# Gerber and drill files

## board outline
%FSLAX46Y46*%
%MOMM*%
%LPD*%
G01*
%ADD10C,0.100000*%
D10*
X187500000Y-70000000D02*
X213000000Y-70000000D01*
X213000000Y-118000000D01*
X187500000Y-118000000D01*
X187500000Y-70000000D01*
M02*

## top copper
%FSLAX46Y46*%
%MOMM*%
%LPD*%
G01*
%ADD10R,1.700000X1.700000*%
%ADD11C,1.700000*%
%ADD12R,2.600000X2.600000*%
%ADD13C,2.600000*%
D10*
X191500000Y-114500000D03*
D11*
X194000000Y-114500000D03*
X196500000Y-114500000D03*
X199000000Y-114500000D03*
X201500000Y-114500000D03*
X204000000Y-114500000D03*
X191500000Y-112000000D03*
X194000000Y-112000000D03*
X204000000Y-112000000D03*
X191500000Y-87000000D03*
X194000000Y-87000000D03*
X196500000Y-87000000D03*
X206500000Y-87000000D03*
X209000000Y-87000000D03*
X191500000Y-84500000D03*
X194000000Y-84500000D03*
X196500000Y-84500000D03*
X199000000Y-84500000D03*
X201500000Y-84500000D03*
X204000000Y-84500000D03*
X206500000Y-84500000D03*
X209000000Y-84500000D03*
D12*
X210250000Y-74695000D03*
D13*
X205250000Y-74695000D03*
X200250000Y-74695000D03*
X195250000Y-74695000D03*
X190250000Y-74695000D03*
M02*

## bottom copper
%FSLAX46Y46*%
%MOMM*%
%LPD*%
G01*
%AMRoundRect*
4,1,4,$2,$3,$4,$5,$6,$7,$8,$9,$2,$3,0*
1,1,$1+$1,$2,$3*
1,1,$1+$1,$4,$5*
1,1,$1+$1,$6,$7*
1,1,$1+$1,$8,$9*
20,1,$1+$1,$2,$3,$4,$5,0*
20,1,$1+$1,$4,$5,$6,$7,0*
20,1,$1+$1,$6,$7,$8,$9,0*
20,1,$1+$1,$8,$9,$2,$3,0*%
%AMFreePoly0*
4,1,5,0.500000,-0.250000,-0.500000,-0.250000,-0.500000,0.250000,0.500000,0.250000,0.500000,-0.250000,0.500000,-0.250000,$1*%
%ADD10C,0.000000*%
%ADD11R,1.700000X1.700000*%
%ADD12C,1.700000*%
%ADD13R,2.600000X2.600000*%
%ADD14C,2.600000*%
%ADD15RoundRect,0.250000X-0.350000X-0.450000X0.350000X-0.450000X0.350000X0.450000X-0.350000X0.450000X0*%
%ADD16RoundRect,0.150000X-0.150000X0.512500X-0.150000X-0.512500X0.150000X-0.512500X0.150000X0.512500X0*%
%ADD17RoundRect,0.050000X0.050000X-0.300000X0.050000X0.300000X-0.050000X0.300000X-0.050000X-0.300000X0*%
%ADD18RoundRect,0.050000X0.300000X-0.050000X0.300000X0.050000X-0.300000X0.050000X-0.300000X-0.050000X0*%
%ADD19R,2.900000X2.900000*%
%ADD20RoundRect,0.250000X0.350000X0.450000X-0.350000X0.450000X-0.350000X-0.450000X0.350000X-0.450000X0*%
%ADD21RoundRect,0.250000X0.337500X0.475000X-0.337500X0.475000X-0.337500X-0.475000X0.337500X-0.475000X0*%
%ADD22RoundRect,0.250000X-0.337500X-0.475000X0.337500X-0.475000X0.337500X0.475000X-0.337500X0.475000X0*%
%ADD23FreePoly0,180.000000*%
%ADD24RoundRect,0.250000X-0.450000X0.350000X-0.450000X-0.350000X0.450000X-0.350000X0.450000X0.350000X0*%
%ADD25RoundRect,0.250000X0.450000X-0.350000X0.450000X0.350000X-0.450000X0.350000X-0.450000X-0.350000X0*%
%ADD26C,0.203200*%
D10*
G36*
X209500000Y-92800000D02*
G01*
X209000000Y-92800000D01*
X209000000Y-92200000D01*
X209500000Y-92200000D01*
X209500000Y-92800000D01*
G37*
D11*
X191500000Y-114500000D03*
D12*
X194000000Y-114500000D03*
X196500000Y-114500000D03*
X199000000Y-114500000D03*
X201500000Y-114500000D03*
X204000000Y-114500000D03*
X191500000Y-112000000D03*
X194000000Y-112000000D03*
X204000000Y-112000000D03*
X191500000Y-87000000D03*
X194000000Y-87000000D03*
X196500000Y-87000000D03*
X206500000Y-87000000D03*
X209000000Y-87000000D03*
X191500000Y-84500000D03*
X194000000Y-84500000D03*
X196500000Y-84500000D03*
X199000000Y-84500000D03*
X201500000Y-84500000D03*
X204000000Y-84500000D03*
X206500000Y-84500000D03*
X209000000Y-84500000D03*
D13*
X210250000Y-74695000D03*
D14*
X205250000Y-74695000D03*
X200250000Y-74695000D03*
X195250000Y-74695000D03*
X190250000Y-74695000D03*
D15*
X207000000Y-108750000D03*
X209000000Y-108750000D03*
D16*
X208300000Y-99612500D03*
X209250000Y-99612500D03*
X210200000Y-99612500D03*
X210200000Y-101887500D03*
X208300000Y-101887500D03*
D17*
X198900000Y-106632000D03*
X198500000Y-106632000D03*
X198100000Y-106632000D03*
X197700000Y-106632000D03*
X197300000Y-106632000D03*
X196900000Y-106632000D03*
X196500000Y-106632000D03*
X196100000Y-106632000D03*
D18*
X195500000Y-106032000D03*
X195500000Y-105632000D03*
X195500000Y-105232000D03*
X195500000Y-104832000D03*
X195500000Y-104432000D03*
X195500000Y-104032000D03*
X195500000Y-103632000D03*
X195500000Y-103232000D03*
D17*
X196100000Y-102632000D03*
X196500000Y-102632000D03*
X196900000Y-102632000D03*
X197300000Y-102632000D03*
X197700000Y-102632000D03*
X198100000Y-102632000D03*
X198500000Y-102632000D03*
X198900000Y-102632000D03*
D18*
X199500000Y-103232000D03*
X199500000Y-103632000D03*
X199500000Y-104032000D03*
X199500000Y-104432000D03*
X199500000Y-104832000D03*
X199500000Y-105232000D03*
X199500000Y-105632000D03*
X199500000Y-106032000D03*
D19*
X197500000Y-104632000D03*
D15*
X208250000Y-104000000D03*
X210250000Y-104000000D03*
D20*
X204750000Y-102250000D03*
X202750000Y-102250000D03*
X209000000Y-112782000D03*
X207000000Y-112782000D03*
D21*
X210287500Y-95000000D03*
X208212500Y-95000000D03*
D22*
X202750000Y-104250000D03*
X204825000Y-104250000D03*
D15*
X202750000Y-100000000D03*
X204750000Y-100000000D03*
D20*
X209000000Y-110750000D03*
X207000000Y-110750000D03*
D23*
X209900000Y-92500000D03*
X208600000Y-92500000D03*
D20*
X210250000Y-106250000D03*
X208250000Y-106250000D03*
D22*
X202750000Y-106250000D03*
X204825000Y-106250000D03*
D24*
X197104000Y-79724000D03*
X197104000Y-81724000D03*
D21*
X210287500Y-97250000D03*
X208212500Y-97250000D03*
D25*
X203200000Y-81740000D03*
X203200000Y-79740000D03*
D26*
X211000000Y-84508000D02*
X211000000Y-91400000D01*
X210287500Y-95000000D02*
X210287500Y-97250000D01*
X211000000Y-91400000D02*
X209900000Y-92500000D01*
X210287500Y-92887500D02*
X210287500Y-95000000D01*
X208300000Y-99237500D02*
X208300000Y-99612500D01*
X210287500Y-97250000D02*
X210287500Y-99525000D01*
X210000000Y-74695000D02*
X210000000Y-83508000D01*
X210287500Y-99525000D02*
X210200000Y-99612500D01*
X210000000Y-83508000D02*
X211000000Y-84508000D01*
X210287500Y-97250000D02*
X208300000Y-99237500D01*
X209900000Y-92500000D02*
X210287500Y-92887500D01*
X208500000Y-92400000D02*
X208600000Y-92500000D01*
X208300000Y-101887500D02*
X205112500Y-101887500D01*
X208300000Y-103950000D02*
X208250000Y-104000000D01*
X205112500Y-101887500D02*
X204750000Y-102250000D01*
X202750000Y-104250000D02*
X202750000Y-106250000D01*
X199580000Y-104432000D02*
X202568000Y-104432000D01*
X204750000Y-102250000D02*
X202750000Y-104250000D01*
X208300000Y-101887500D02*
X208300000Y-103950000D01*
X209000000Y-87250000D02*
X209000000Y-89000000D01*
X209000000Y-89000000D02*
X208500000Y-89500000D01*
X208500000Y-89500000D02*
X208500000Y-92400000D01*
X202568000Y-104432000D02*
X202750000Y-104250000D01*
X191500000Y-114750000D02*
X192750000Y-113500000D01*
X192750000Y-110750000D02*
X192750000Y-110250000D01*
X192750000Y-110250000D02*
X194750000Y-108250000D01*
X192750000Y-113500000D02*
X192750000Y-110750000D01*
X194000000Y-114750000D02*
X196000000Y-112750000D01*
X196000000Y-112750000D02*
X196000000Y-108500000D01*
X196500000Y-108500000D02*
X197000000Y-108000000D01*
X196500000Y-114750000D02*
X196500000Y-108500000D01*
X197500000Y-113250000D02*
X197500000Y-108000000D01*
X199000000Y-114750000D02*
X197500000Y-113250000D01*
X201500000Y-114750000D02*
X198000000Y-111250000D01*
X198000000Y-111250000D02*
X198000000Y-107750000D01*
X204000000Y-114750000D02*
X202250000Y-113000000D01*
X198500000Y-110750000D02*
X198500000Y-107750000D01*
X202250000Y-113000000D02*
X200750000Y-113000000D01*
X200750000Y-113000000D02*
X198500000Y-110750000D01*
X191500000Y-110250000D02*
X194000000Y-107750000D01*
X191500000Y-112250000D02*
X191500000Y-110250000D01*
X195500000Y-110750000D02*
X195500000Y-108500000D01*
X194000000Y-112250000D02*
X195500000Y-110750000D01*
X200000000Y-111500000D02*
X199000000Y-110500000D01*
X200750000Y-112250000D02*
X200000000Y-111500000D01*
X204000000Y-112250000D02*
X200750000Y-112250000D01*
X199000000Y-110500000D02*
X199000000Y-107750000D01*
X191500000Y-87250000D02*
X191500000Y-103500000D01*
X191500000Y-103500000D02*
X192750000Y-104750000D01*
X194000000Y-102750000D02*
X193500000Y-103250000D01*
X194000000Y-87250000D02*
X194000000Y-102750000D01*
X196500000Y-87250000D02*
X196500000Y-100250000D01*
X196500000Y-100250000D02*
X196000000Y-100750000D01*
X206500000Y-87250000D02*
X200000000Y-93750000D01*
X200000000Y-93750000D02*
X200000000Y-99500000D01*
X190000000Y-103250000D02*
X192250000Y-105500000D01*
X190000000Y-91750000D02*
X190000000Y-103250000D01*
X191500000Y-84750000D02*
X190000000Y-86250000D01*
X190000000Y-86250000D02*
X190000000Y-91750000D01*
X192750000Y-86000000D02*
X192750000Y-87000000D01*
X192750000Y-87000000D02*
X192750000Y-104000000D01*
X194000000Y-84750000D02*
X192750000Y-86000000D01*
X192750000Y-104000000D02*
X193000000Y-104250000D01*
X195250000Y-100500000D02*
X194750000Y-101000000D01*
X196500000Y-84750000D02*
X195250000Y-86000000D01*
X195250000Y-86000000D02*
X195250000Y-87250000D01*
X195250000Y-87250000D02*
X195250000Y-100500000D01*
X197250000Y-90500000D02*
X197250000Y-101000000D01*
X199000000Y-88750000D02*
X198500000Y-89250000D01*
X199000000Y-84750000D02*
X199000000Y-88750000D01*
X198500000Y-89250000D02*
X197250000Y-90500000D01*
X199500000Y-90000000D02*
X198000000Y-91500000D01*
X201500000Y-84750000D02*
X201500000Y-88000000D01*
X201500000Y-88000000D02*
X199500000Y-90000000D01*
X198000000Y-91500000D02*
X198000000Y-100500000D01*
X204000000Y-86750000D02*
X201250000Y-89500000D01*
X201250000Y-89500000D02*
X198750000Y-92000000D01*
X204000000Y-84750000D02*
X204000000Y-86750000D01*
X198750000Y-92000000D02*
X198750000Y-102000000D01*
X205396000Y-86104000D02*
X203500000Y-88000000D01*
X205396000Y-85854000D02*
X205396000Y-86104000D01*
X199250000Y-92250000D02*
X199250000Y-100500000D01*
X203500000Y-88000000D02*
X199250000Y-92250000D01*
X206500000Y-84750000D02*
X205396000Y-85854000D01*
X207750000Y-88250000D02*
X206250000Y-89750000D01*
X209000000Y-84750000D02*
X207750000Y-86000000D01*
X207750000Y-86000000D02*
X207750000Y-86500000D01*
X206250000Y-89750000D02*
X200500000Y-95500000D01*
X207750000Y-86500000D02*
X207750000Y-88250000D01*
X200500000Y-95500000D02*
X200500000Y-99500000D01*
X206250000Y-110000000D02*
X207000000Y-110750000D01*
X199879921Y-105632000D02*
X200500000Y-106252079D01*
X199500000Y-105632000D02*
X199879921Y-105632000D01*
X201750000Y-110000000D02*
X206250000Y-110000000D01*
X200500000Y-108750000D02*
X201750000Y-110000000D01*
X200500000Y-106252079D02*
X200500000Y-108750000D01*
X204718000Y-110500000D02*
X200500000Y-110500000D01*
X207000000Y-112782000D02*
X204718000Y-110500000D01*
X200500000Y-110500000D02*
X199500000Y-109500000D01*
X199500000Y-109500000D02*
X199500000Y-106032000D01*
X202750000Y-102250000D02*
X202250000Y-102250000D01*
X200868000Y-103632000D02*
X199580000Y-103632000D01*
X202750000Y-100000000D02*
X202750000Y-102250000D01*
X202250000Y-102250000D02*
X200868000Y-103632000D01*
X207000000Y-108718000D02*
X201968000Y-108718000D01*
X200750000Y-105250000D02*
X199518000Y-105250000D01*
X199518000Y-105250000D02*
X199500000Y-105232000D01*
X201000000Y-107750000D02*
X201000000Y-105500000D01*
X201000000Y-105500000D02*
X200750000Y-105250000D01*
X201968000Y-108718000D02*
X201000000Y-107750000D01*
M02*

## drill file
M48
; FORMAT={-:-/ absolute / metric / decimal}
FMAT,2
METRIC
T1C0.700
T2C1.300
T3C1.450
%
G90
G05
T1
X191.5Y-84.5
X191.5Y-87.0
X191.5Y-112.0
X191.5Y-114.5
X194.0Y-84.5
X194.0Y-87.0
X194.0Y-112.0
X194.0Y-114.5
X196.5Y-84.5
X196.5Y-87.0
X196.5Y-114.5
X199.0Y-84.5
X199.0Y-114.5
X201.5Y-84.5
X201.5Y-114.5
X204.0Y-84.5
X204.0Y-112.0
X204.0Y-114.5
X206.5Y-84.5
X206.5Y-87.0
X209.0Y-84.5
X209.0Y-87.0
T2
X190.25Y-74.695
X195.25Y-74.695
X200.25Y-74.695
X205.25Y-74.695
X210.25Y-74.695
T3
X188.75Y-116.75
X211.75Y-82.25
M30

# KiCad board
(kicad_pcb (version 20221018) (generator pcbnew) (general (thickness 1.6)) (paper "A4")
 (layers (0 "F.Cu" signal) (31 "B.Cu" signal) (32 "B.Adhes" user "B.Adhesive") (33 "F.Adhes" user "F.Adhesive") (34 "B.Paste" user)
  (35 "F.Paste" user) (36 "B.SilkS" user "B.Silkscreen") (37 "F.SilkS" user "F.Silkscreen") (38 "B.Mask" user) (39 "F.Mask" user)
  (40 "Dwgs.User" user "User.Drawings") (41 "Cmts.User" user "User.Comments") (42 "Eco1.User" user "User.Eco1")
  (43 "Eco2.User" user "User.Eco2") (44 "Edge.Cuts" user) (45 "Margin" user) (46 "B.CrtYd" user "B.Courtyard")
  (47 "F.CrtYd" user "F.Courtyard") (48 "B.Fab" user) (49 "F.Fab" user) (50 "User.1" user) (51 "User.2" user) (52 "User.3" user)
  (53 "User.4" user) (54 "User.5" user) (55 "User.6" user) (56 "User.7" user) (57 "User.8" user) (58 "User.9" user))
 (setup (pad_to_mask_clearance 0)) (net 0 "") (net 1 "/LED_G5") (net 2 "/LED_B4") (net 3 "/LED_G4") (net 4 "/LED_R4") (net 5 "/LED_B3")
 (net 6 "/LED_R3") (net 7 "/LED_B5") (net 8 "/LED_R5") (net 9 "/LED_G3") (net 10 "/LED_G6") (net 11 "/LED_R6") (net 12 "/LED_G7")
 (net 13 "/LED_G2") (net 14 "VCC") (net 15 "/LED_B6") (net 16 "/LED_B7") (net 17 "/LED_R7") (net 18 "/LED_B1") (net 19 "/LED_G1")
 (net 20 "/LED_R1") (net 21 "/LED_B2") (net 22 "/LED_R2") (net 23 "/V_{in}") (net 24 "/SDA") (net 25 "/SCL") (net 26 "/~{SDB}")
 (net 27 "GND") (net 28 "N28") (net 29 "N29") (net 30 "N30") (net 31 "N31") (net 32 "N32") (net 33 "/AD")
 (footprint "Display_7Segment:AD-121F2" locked (layer "F.Cu") (at 191.5 114.5 90)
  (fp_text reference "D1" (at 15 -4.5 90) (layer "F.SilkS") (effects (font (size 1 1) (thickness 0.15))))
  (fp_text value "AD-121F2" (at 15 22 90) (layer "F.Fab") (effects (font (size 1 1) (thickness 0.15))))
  (pad "" np_thru_hole circle locked (at -2.25 -2.75 90) (size 1.45 1.45) (drill 1.45) (layers "*.Cu" "*.Mask"))
  (pad "" np_thru_hole circle locked (at 32.25 20.25 90) (size 1.45 1.45) (drill 1.45) (layers "*.Cu" "*.Mask"))
  (pad "1" thru_hole rect locked (at 0 0 90) (size 1.7 1.7) (drill 0.7) (layers "*.Cu" "*.Mask") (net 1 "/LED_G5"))
  (pad "2" thru_hole circle locked (at 0 2.5 90) (size 1.7 1.7) (drill 0.7) (layers "*.Cu" "*.Mask") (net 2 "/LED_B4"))
  (pad "3" thru_hole circle locked (at 0 5 90) (size 1.7 1.7) (drill 0.7) (layers "*.Cu" "*.Mask") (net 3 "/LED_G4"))
  (pad "4" thru_hole circle locked (at 0 7.5 90) (size 1.7 1.7) (drill 0.7) (layers "*.Cu" "*.Mask") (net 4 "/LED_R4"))
  (pad "5" thru_hole circle locked (at 0 10 90) (size 1.7 1.7) (drill 0.7) (layers "*.Cu" "*.Mask") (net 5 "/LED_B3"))
  (pad "6" thru_hole circle locked (at 0 12.5 90) (size 1.7 1.7) (drill 0.7) (layers "*.Cu" "*.Mask") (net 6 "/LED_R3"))
  (pad "9" thru_hole circle locked (at 2.5 0 90) (size 1.7 1.7) (drill 0.7) (layers "*.Cu" "*.Mask") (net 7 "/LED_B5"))
  (pad "10" thru_hole circle locked (at 2.5 2.5 90) (size 1.7 1.7) (drill 0.7) (layers "*.Cu" "*.Mask") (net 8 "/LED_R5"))
  (pad "11" thru_hole circle locked (at 2.5 12.5 90) (size 1.7 1.7) (drill 0.7) (layers "*.Cu" "*.Mask") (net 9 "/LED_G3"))
  (pad "13" thru_hole circle locked (at 27.5 0 90) (size 1.7 1.7) (drill 0.7) (layers "*.Cu" "*.Mask") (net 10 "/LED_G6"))
  (pad "14" thru_hole circle locked (at 27.5 2.5 90) (size 1.7 1.7) (drill 0.7) (layers "*.Cu" "*.Mask") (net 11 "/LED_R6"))
  (pad "15" thru_hole circle locked (at 27.5 5 90) (size 1.7 1.7) (drill 0.7) (layers "*.Cu" "*.Mask") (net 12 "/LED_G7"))
  (pad "16" thru_hole circle locked (at 27.5 15 90) (size 1.7 1.7) (drill 0.7) (layers "*.Cu" "*.Mask") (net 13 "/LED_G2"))
  (pad "17" thru_hole circle locked (at 27.5 17.5 90) (size 1.7 1.7) (drill 0.7) (layers "*.Cu" "*.Mask") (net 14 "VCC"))
  (pad "18" thru_hole circle locked (at 30 0 90) (size 1.7 1.7) (drill 0.7) (layers "*.Cu" "*.Mask") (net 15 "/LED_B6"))
  (pad "19" thru_hole circle locked (at 30 2.5 90) (size 1.7 1.7) (drill 0.7) (layers "*.Cu" "*.Mask") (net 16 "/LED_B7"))
  (pad "20" thru_hole circle locked (at 30 5 90) (size 1.7 1.7) (drill 0.7) (layers "*.Cu" "*.Mask") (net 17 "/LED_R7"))
  (pad "21" thru_hole circle locked (at 30 7.5 90) (size 1.7 1.7) (drill 0.7) (layers "*.Cu" "*.Mask") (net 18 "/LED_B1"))
  (pad "22" thru_hole circle locked (at 30 10 90) (size 1.7 1.7) (drill 0.7) (layers "*.Cu" "*.Mask") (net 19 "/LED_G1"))
  (pad "23" thru_hole circle locked (at 30 12.5 90) (size 1.7 1.7) (drill 0.7) (layers "*.Cu" "*.Mask") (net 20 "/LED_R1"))
  (pad "24" thru_hole circle locked (at 30 15 90) (size 1.7 1.7) (drill 0.7) (layers "*.Cu" "*.Mask") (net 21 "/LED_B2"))
  (pad "25" thru_hole circle locked (at 30 17.5 90) (size 1.7 1.7) (drill 0.7) (layers "*.Cu" "*.Mask") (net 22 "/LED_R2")))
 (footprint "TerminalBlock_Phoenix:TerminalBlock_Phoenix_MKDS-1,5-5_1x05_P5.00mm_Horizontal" (layer "F.Cu") (at 210.25 74.695 180)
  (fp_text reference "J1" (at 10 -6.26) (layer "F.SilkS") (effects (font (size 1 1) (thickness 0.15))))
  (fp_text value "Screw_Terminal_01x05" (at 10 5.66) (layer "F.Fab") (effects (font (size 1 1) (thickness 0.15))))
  (pad "1" thru_hole rect (at 0 0 180) (size 2.6 2.6) (drill 1.3) (layers "*.Cu" "*.Mask") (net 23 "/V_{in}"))
  (pad "2" thru_hole circle (at 5 0 180) (size 2.6 2.6) (drill 1.3) (layers "*.Cu" "*.Mask") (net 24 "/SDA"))
  (pad "3" thru_hole circle (at 10 0 180) (size 2.6 2.6) (drill 1.3) (layers "*.Cu" "*.Mask") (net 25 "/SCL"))
  (pad "4" thru_hole circle (at 15 0 180) (size 2.6 2.6) (drill 1.3) (layers "*.Cu" "*.Mask") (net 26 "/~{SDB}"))
  (pad "5" thru_hole circle (at 20 0 180) (size 2.6 2.6) (drill 1.3) (layers "*.Cu" "*.Mask") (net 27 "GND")))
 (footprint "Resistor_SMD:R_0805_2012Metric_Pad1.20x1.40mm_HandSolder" (layer "B.Cu") (at 208 108.75)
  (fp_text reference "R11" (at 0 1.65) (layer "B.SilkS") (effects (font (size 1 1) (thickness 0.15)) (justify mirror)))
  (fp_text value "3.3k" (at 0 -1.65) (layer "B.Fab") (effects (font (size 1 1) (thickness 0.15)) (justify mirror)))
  (pad "1" smd roundrect (at -1 0) (size 1.2 1.4) (layers "B.Cu" "B.Paste" "B.Mask") (roundrect_rratio 0.208333) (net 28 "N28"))
  (pad "2" smd roundrect (at 1 0) (size 1.2 1.4) (layers "B.Cu" "B.Paste" "B.Mask") (roundrect_rratio 0.208333) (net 27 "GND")))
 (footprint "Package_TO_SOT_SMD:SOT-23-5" (layer "B.Cu") (at 209.25 100.75 -90)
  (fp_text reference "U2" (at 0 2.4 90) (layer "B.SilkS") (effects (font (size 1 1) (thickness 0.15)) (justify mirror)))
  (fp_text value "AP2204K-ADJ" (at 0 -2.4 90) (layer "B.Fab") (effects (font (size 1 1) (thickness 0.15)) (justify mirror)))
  (pad "1" smd roundrect (at -1.1375 0.95 270) (size 1.325 0.6) (layers "B.Cu" "B.Paste" "B.Mask") (roundrect_rratio 0.25)
   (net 23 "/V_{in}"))
  (pad "2" smd roundrect (at -1.1375 0 270) (size 1.325 0.6) (layers "B.Cu" "B.Paste" "B.Mask") (roundrect_rratio 0.25) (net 27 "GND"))
  (pad "3" smd roundrect (at -1.1375 -0.95 270) (size 1.325 0.6) (layers "B.Cu" "B.Paste" "B.Mask") (roundrect_rratio 0.25)
   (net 23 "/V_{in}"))
  (pad "4" smd roundrect (at 1.1375 -0.95 270) (size 1.325 0.6) (layers "B.Cu" "B.Paste" "B.Mask") (roundrect_rratio 0.25) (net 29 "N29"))
  (pad "5" smd roundrect (at 1.1375 0.95 270) (size 1.325 0.6) (layers "B.Cu" "B.Paste" "B.Mask") (roundrect_rratio 0.25) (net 14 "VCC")))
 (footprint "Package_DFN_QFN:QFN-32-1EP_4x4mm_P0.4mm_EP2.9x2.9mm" (layer "B.Cu") (at 197.5 104.632 90)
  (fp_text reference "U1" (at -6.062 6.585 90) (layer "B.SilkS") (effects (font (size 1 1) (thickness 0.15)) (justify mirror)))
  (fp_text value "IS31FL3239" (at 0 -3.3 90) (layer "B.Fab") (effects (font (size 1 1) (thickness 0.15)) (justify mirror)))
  (pad "" smd roundrect (at -0.725 -0.725 90) (size 1.17 1.17) (layers "B.Paste") (roundrect_rratio 0.213675))
  (pad "" smd roundrect (at -0.725 0.725 90) (size 1.17 1.17) (layers "B.Paste") (roundrect_rratio 0.213675))
  (pad "" smd roundrect (at 0.725 -0.725 90) (size 1.17 1.17) (layers "B.Paste") (roundrect_rratio 0.213675))
  (pad "" smd roundrect (at 0.725 0.725 90) (size 1.17 1.17) (layers "B.Paste") (roundrect_rratio 0.213675))
  (pad "1" smd roundrect (at -2 1.4 90) (size 0.7 0.2) (layers "B.Cu" "B.Paste" "B.Mask") (roundrect_rratio 0.25) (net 20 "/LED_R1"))
  (pad "2" smd roundrect (at -2 1 90) (size 0.7 0.2) (layers "B.Cu" "B.Paste" "B.Mask") (roundrect_rratio 0.25) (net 19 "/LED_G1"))
  (pad "3" smd roundrect (at -2 0.6 90) (size 0.7 0.2) (layers "B.Cu" "B.Paste" "B.Mask") (roundrect_rratio 0.25) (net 18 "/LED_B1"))
  (pad "4" smd roundrect (at -2 0.2 90) (size 0.7 0.2) (layers "B.Cu" "B.Paste" "B.Mask") (roundrect_rratio 0.25) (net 22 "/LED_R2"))
  (pad "5" smd roundrect (at -2 -0.2 90) (size 0.7 0.2) (layers "B.Cu" "B.Paste" "B.Mask") (roundrect_rratio 0.25) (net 13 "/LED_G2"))
  (pad "6" smd roundrect (at -2 -0.6 90) (size 0.7 0.2) (layers "B.Cu" "B.Paste" "B.Mask") (roundrect_rratio 0.25) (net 21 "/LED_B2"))
  (pad "7" smd roundrect (at -2 -1 90) (size 0.7 0.2) (layers "B.Cu" "B.Paste" "B.Mask") (roundrect_rratio 0.25) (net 6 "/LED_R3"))
  (pad "8" smd roundrect (at -2 -1.4 90) (size 0.7 0.2) (layers "B.Cu" "B.Paste" "B.Mask") (roundrect_rratio 0.25) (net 9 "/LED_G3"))
  (pad "9" smd roundrect (at -1.4 -2 90) (size 0.2 0.7) (layers "B.Cu" "B.Paste" "B.Mask") (roundrect_rratio 0.25) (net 5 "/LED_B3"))
  (pad "10" smd roundrect (at -1 -2 90) (size 0.2 0.7) (layers "B.Cu" "B.Paste" "B.Mask") (roundrect_rratio 0.25) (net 4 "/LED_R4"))
  (pad "11" smd roundrect (at -0.6 -2 90) (size 0.2 0.7) (layers "B.Cu" "B.Paste" "B.Mask") (roundrect_rratio 0.25) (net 3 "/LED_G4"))
  (pad "12" smd roundrect (at -0.2 -2 90) (size 0.2 0.7) (layers "B.Cu" "B.Paste" "B.Mask") (roundrect_rratio 0.25) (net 2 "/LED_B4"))
  (pad "13" smd roundrect (at 0.2 -2 90) (size 0.2 0.7) (layers "B.Cu" "B.Paste" "B.Mask") (roundrect_rratio 0.25) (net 27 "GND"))
  (pad "14" smd roundrect (at 0.6 -2 90) (size 0.2 0.7) (layers "B.Cu" "B.Paste" "B.Mask") (roundrect_rratio 0.25) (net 8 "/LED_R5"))
  (pad "15" smd roundrect (at 1 -2 90) (size 0.2 0.7) (layers "B.Cu" "B.Paste" "B.Mask") (roundrect_rratio 0.25) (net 1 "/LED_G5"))
  (pad "16" smd roundrect (at 1.4 -2 90) (size 0.2 0.7) (layers "B.Cu" "B.Paste" "B.Mask") (roundrect_rratio 0.25) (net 7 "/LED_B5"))
  (pad "17" smd roundrect (at 2 -1.4 90) (size 0.7 0.2) (layers "B.Cu" "B.Paste" "B.Mask") (roundrect_rratio 0.25) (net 11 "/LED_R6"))
  (pad "18" smd roundrect (at 2 -1 90) (size 0.7 0.2) (layers "B.Cu" "B.Paste" "B.Mask") (roundrect_rratio 0.25) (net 10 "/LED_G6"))
  (pad "19" smd roundrect (at 2 -0.6 90) (size 0.7 0.2) (layers "B.Cu" "B.Paste" "B.Mask") (roundrect_rratio 0.25) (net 15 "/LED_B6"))
  (pad "20" smd roundrect (at 2 -0.2 90) (size 0.7 0.2) (layers "B.Cu" "B.Paste" "B.Mask") (roundrect_rratio 0.25) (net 17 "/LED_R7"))
  (pad "21" smd roundrect (at 2 0.2 90) (size 0.7 0.2) (layers "B.Cu" "B.Paste" "B.Mask") (roundrect_rratio 0.25) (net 12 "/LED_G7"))
  (pad "22" smd roundrect (at 2 0.6 90) (size 0.7 0.2) (layers "B.Cu" "B.Paste" "B.Mask") (roundrect_rratio 0.25) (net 16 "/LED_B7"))
  (pad "23" smd roundrect (at 2 1 90) (size 0.7 0.2) (layers "B.Cu" "B.Paste" "B.Mask") (roundrect_rratio 0.25) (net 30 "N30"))
  (pad "24" smd roundrect (at 2 1.4 90) (size 0.7 0.2) (layers "B.Cu" "B.Paste" "B.Mask") (roundrect_rratio 0.25) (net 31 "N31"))
  (pad "25" smd roundrect (at 1.4 2 90) (size 0.2 0.7) (layers "B.Cu" "B.Paste" "B.Mask") (roundrect_rratio 0.25) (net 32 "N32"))
  (pad "26" smd roundrect (at 1 2 90) (size 0.2 0.7) (layers "B.Cu" "B.Paste" "B.Mask") (roundrect_rratio 0.25) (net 26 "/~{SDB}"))
  (pad "27" smd roundrect (at 0.6 2 90) (size 0.2 0.7) (layers "B.Cu" "B.Paste" "B.Mask") (roundrect_rratio 0.25) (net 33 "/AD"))
  (pad "28" smd roundrect (at 0.2 2 90) (size 0.2 0.7) (layers "B.Cu" "B.Paste" "B.Mask") (roundrect_rratio 0.25) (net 14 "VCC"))
  (pad "29" smd roundrect (at -0.2 2 90) (size 0.2 0.7) (layers "B.Cu" "B.Paste" "B.Mask") (roundrect_rratio 0.25) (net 27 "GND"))
  (pad "30" smd roundrect (at -0.6 2 90) (size 0.2 0.7) (layers "B.Cu" "B.Paste" "B.Mask") (roundrect_rratio 0.25) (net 28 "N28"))
  (pad "31" smd roundrect (at -1 2 90) (size 0.2 0.7) (layers "B.Cu" "B.Paste" "B.Mask") (roundrect_rratio 0.25) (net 24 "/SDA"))
  (pad "32" smd roundrect (at -1.4 2 90) (size 0.2 0.7) (layers "B.Cu" "B.Paste" "B.Mask") (roundrect_rratio 0.25) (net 25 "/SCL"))
  (pad "33" smd rect (at 0 0 90) (size 2.9 2.9) (layers "B.Cu" "B.Mask") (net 27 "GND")))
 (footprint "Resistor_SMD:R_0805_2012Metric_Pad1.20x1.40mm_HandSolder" (layer "B.Cu") (at 209.25 104)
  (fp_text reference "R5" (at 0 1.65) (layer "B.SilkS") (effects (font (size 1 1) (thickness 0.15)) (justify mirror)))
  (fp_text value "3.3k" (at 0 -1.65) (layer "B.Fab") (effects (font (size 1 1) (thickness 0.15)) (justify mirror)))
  (pad "1" smd roundrect (at -1 0) (size 1.2 1.4) (layers "B.Cu" "B.Paste" "B.Mask") (roundrect_rratio 0.208333) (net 14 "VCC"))
  (pad "2" smd roundrect (at 1 0) (size 1.2 1.4) (layers "B.Cu" "B.Paste" "B.Mask") (roundrect_rratio 0.208333) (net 29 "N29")))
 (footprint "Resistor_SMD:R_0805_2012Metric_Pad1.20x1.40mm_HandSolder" (layer "B.Cu") (at 203.75 102.25 180)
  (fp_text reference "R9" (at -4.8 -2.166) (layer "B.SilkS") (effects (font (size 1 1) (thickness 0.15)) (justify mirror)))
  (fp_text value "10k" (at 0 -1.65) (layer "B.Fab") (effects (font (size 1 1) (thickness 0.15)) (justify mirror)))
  (pad "1" smd roundrect (at -1 0 180) (size 1.2 1.4) (layers "B.Cu" "B.Paste" "B.Mask") (roundrect_rratio 0.208333) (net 14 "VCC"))
  (pad "2" smd roundrect (at 1 0 180) (size 1.2 1.4) (layers "B.Cu" "B.Paste" "B.Mask") (roundrect_rratio 0.208333) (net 26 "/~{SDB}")))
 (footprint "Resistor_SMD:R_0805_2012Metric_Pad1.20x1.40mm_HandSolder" (layer "B.Cu") (at 208 112.782 180)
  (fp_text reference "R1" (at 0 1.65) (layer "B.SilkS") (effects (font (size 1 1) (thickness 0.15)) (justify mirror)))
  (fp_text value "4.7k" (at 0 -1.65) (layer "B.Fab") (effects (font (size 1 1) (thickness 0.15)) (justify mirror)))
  (pad "1" smd roundrect (at -1 0 180) (size 1.2 1.4) (layers "B.Cu" "B.Paste" "B.Mask") (roundrect_rratio 0.208333) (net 14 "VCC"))
  (pad "2" smd roundrect (at 1 0 180) (size 1.2 1.4) (layers "B.Cu" "B.Paste" "B.Mask") (roundrect_rratio 0.208333) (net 25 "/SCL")))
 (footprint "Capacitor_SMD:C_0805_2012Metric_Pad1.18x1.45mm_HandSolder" (layer "B.Cu") (at 209.25 95 180)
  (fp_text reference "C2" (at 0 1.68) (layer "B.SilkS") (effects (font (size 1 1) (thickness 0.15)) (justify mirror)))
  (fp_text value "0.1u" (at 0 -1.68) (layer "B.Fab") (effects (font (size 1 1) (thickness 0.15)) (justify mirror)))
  (pad "1" smd roundrect (at -1.0375 0 180) (size 1.175 1.45) (layers "B.Cu" "B.Paste" "B.Mask") (roundrect_rratio 0.212766)
   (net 23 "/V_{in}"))
  (pad "2" smd roundrect (at 1.0375 0 180) (size 1.175 1.45) (layers "B.Cu" "B.Paste" "B.Mask") (roundrect_rratio 0.212766) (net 27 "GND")))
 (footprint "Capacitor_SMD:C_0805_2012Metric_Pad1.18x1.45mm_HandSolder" (layer "B.Cu") (at 203.7875 104.25)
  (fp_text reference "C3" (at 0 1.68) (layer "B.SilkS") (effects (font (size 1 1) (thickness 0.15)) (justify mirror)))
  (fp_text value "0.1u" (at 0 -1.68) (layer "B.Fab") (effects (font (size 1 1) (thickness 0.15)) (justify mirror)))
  (pad "1" smd roundrect (at -1.0375 0) (size 1.175 1.45) (layers "B.Cu" "B.Paste" "B.Mask") (roundrect_rratio 0.212766) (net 14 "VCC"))
  (pad "2" smd roundrect (at 1.0375 0) (size 1.175 1.45) (layers "B.Cu" "B.Paste" "B.Mask") (roundrect_rratio 0.212766) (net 27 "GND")))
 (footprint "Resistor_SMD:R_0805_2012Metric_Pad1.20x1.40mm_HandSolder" (layer "B.Cu") (at 203.75 100)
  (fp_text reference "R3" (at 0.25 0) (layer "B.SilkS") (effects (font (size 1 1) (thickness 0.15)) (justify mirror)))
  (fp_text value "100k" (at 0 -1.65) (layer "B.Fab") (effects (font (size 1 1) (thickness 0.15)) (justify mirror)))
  (pad "1" smd roundrect (at -1 0) (size 1.2 1.4) (layers "B.Cu" "B.Paste" "B.Mask") (roundrect_rratio 0.208333) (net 26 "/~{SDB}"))
  (pad "2" smd roundrect (at 1 0) (size 1.2 1.4) (layers "B.Cu" "B.Paste" "B.Mask") (roundrect_rratio 0.208333) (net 27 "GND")))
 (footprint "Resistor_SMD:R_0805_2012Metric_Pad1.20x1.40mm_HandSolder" (layer "B.Cu") (at 208 110.75 180)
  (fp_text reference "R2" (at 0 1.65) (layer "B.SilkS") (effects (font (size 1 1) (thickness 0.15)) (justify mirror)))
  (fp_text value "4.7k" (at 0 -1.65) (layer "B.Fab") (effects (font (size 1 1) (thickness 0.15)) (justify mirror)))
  (pad "1" smd roundrect (at -1 0 180) (size 1.2 1.4) (layers "B.Cu" "B.Paste" "B.Mask") (roundrect_rratio 0.208333) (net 14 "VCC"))
  (pad "2" smd roundrect (at 1 0 180) (size 1.2 1.4) (layers "B.Cu" "B.Paste" "B.Mask") (roundrect_rratio 0.208333) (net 24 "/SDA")))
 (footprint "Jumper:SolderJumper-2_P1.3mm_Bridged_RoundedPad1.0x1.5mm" (layer "B.Cu") (at 209.25 92.5 180) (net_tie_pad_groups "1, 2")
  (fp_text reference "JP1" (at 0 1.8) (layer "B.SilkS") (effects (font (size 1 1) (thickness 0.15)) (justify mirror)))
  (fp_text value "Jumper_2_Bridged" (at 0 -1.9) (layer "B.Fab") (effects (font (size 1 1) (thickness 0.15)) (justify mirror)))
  (fp_poly (pts (xy 0.25 0.3) (xy -0.25 0.3) (xy -0.25 -0.3) (xy 0.25 -0.3)) (stroke (width 0) (type solid)) (fill solid) (layer "B.Cu"))
  (pad "1" smd custom (at -0.65 0 180) (size 1 0.5) (layers "B.Cu" "B.Mask") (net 23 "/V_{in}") (zone_connect 2) (thermal_bridge_angle 45)
   (options (clearance outline) (anchor rect)) (primitives))
  (pad "2" smd custom (at 0.65 0 180) (size 1 0.5) (layers "B.Cu" "B.Mask") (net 14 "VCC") (zone_connect 2) (thermal_bridge_angle 45)
   (options (clearance outline) (anchor rect)) (primitives)))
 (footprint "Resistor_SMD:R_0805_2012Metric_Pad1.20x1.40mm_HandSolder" (layer "B.Cu") (at 209.25 106.25 180)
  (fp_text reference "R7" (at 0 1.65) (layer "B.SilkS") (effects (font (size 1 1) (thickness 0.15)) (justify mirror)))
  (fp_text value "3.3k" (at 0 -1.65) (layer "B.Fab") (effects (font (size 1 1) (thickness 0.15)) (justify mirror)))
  (pad "1" smd roundrect (at -1 0 180) (size 1.2 1.4) (layers "B.Cu" "B.Paste" "B.Mask") (roundrect_rratio 0.208333) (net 27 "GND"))
  (pad "2" smd roundrect (at 1 0 180) (size 1.2 1.4) (layers "B.Cu" "B.Paste" "B.Mask") (roundrect_rratio 0.208333) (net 29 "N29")))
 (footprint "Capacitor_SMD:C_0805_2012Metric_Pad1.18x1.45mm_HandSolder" (layer "B.Cu") (at 203.7875 106.25)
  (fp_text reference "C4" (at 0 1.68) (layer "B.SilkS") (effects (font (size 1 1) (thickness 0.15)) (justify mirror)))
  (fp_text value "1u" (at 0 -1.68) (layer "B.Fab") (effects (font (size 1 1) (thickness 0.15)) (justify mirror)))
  (pad "1" smd roundrect (at -1.0375 0) (size 1.175 1.45) (layers "B.Cu" "B.Paste" "B.Mask") (roundrect_rratio 0.212766) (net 14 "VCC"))
  (pad "2" smd roundrect (at 1.0375 0) (size 1.175 1.45) (layers "B.Cu" "B.Paste" "B.Mask") (roundrect_rratio 0.212766) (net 27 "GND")))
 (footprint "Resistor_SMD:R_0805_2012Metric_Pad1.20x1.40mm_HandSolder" (layer "B.Cu") (at 197.104 80.724 -90)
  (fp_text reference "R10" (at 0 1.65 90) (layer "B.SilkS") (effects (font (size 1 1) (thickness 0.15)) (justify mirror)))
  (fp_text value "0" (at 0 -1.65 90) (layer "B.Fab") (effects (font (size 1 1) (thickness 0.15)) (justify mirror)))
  (pad "1" smd roundrect (at -1 0 270) (size 1.2 1.4) (layers "B.Cu" "B.Paste" "B.Mask") (roundrect_rratio 0.208333) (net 27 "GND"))
  (pad "2" smd roundrect (at 1 0 270) (size 1.2 1.4) (layers "B.Cu" "B.Paste" "B.Mask") (roundrect_rratio 0.208333) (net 33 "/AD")))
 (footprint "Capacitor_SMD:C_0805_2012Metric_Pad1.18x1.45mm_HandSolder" (layer "B.Cu") (at 209.25 97.25 180)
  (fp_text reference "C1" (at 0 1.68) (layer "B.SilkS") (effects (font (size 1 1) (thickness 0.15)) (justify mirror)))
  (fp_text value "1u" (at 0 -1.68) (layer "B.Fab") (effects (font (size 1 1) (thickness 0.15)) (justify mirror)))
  (pad "1" smd roundrect (at -1.0375 0 180) (size 1.175 1.45) (layers "B.Cu" "B.Paste" "B.Mask") (roundrect_rratio 0.212766)
   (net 23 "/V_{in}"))
  (pad "2" smd roundrect (at 1.0375 0 180) (size 1.175 1.45) (layers "B.Cu" "B.Paste" "B.Mask") (roundrect_rratio 0.212766) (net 27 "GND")))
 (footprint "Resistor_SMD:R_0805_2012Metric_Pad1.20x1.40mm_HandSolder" (layer "B.Cu") (at 203.2 80.74 90)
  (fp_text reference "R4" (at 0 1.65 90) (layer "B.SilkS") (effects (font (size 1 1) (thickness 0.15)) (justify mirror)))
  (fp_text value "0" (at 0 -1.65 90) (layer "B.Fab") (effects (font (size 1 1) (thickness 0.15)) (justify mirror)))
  (pad "1" smd roundrect (at -1 0 90) (size 1.2 1.4) (layers "B.Cu" "B.Paste" "B.Mask") (roundrect_rratio 0.208333) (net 14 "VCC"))
  (pad "2" smd roundrect (at 1 0 90) (size 1.2 1.4) (layers "B.Cu" "B.Paste" "B.Mask") (roundrect_rratio 0.208333) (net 33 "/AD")))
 (gr_rect (start 187.5 70) (end 213 118) (stroke (width 0.1) (type default)) (fill none) (layer "Edge.Cuts"))
 (segment (start 211 84.508) (end 211 91.4) (width 0.2032) (layer "B.Cu") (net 23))
 (segment (start 210.2875 95) (end 210.2875 97.25) (width 0.2032) (layer "B.Cu") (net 23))
 (segment (start 211 91.4) (end 209.9 92.5) (width 0.2032) (layer "B.Cu") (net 23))
 (segment (start 210.2875 92.8875) (end 210.2875 95) (width 0.2032) (layer "B.Cu") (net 23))
 (segment (start 208.3 99.2375) (end 208.3 99.6125) (width 0.2032) (layer "B.Cu") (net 23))
 (segment (start 210.2875 97.25) (end 210.2875 99.525) (width 0.2032) (layer "B.Cu") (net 23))
 (segment (start 210 74.695) (end 210 83.508) (width 0.2032) (layer "B.Cu") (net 23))
 (segment (start 210.2875 99.525) (end 210.2 99.6125) (width 0.2032) (layer "B.Cu") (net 23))
 (segment (start 210 83.508) (end 211 84.508) (width 0.2032) (layer "B.Cu") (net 23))
 (segment (start 210.2875 97.25) (end 208.3 99.2375) (width 0.2032) (layer "B.Cu") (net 23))
 (segment (start 209.9 92.5) (end 210.2875 92.8875) (width 0.2032) (layer "B.Cu") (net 23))
 (segment (start 208.5 92.4) (end 208.6 92.5) (width 0.2032) (layer "B.Cu") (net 14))
 (segment (start 208.3 101.8875) (end 205.1125 101.8875) (width 0.2032) (layer "B.Cu") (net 14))
 (segment (start 208.3 103.95) (end 208.25 104) (width 0.2032) (layer "B.Cu") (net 14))
 (segment (start 205.1125 101.8875) (end 204.75 102.25) (width 0.2032) (layer "B.Cu") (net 14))
 (segment (start 202.75 104.25) (end 202.75 106.25) (width 0.2032) (layer "B.Cu") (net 14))
 (segment (start 199.58 104.432) (end 202.568 104.432) (width 0.2032) (layer "B.Cu") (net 14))
 (segment (start 204.75 102.25) (end 202.75 104.25) (width 0.2032) (layer "B.Cu") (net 14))
 (segment (start 208.3 101.8875) (end 208.3 103.95) (width 0.2032) (layer "B.Cu") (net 14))
 (segment (start 209 87.25) (end 209 89) (width 0.2032) (layer "B.Cu") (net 14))
 (segment (start 209 89) (end 208.5 89.5) (width 0.2032) (layer "B.Cu") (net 14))
 (segment (start 208.5 89.5) (end 208.5 92.4) (width 0.2032) (layer "B.Cu") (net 14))
 (segment (start 202.568 104.432) (end 202.75 104.25) (width 0.2032) (layer "B.Cu") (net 14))
 (segment (start 191.5 114.75) (end 192.75 113.5) (width 0.2032) (layer "B.Cu") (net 1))
 (segment (start 192.75 110.75) (end 192.75 110.25) (width 0.2032) (layer "B.Cu") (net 1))
 (segment (start 192.75 110.25) (end 194.75 108.25) (width 0.2032) (layer "B.Cu") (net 1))
 (segment (start 192.75 113.5) (end 192.75 110.75) (width 0.2032) (layer "B.Cu") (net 1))
 (segment (start 194 114.75) (end 196 112.75) (width 0.2032) (layer "B.Cu") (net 2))
 (segment (start 196 112.75) (end 196 108.5) (width 0.2032) (layer "B.Cu") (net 2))
 (segment (start 196.5 108.5) (end 197 108) (width 0.2032) (layer "B.Cu") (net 3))
 (segment (start 196.5 114.75) (end 196.5 108.5) (width 0.2032) (layer "B.Cu") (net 3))
 (segment (start 197.5 113.25) (end 197.5 108) (width 0.2032) (layer "B.Cu") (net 4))
 (segment (start 199 114.75) (end 197.5 113.25) (width 0.2032) (layer "B.Cu") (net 4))
 (segment (start 201.5 114.75) (end 198 111.25) (width 0.2032) (layer "B.Cu") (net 5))
 (segment (start 198 111.25) (end 198 107.75) (width 0.2032) (layer "B.Cu") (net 5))
 (segment (start 204 114.75) (end 202.25 113) (width 0.2032) (layer "B.Cu") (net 6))
 (segment (start 198.5 110.75) (end 198.5 107.75) (width 0.2032) (layer "B.Cu") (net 6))
 (segment (start 202.25 113) (end 200.75 113) (width 0.2032) (layer "B.Cu") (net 6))
 (segment (start 200.75 113) (end 198.5 110.75) (width 0.2032) (layer "B.Cu") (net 6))
 (segment (start 191.5 110.25) (end 194 107.75) (width 0.2032) (layer "B.Cu") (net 7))
 (segment (start 191.5 112.25) (end 191.5 110.25) (width 0.2032) (layer "B.Cu") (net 7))
 (segment (start 195.5 110.75) (end 195.5 108.5) (width 0.2032) (layer "B.Cu") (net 8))
 (segment (start 194 112.25) (end 195.5 110.75) (width 0.2032) (layer "B.Cu") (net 8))
 (segment (start 200 111.5) (end 199 110.5) (width 0.2032) (layer "B.Cu") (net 9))
 (segment (start 200.75 112.25) (end 200 111.5) (width 0.2032) (layer "B.Cu") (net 9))
 (segment (start 204 112.25) (end 200.75 112.25) (width 0.2032) (layer "B.Cu") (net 9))
 (segment (start 199 110.5) (end 199 107.75) (width 0.2032) (layer "B.Cu") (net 9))
 (segment (start 191.5 87.25) (end 191.5 103.5) (width 0.2032) (layer "B.Cu") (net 10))
 (segment (start 191.5 103.5) (end 192.75 104.75) (width 0.2032) (layer "B.Cu") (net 10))
 (segment (start 194 102.75) (end 193.5 103.25) (width 0.2032) (layer "B.Cu") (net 11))
 (segment (start 194 87.25) (end 194 102.75) (width 0.2032) (layer "B.Cu") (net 11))
 (segment (start 196.5 87.25) (end 196.5 100.25) (width 0.2032) (layer "B.Cu") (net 12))
 (segment (start 196.5 100.25) (end 196 100.75) (width 0.2032) (layer "B.Cu") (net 12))
 (segment (start 206.5 87.25) (end 200 93.75) (width 0.2032) (layer "B.Cu") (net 13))
 (segment (start 200 93.75) (end 200 99.5) (width 0.2032) (layer "B.Cu") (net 13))
 (segment (start 190 103.25) (end 192.25 105.5) (width 0.2032) (layer "B.Cu") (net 15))
 (segment (start 190 91.75) (end 190 103.25) (width 0.2032) (layer "B.Cu") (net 15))
 (segment (start 191.5 84.75) (end 190 86.25) (width 0.2032) (layer "B.Cu") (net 15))
 (segment (start 190 86.25) (end 190 91.75) (width 0.2032) (layer "B.Cu") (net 15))
 (segment (start 192.75 86) (end 192.75 87) (width 0.2032) (layer "B.Cu") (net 16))
 (segment (start 192.75 87) (end 192.75 104) (width 0.2032) (layer "B.Cu") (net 16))
 (segment (start 194 84.75) (end 192.75 86) (width 0.2032) (layer "B.Cu") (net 16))
 (segment (start 192.75 104) (end 193 104.25) (width 0.2032) (layer "B.Cu") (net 16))
 (segment (start 195.25 100.5) (end 194.75 101) (width 0.2032) (layer "B.Cu") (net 17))
 (segment (start 196.5 84.75) (end 195.25 86) (width 0.2032) (layer "B.Cu") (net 17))
 (segment (start 195.25 86) (end 195.25 87.25) (width 0.2032) (layer "B.Cu") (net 17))
 (segment (start 195.25 87.25) (end 195.25 100.5) (width 0.2032) (layer "B.Cu") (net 17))
 (segment (start 197.25 90.5) (end 197.25 101) (width 0.2032) (layer "B.Cu") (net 18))
 (segment (start 199 88.75) (end 198.5 89.25) (width 0.2032) (layer "B.Cu") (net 18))
 (segment (start 199 84.75) (end 199 88.75) (width 0.2032) (layer "B.Cu") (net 18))
 (segment (start 198.5 89.25) (end 197.25 90.5) (width 0.2032) (layer "B.Cu") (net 18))
 (segment (start 199.5 90) (end 198 91.5) (width 0.2032) (layer "B.Cu") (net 19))
 (segment (start 201.5 84.75) (end 201.5 88) (width 0.2032) (layer "B.Cu") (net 19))
 (segment (start 201.5 88) (end 199.5 90) (width 0.2032) (layer "B.Cu") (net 19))
 (segment (start 198 91.5) (end 198 100.5) (width 0.2032) (layer "B.Cu") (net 19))
 (segment (start 204 86.75) (end 201.25 89.5) (width 0.2032) (layer "B.Cu") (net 20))
 (segment (start 201.25 89.5) (end 198.75 92) (width 0.2032) (layer "B.Cu") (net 20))
 (segment (start 204 84.75) (end 204 86.75) (width 0.2032) (layer "B.Cu") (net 20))
 (segment (start 198.75 92) (end 198.75 102) (width 0.2032) (layer "B.Cu") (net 20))
 (segment (start 205.396 86.104) (end 203.5 88) (width 0.2032) (layer "B.Cu") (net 21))
 (segment (start 205.396 85.854) (end 205.396 86.104) (width 0.2032) (layer "B.Cu") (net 21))
 (segment (start 199.25 92.25) (end 199.25 100.5) (width 0.2032) (layer "B.Cu") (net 21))
 (segment (start 203.5 88) (end 199.25 92.25) (width 0.2032) (layer "B.Cu") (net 21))
 (segment (start 206.5 84.75) (end 205.396 85.854) (width 0.2032) (layer "B.Cu") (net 21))
 (segment (start 207.75 88.25) (end 206.25 89.75) (width 0.2032) (layer "B.Cu") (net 22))
 (segment (start 209 84.75) (end 207.75 86) (width 0.2032) (layer "B.Cu") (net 22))
 (segment (start 207.75 86) (end 207.75 86.5) (width 0.2032) (layer "B.Cu") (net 22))
 (segment (start 206.25 89.75) (end 200.5 95.5) (width 0.2032) (layer "B.Cu") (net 22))
 (segment (start 207.75 86.5) (end 207.75 88.25) (width 0.2032) (layer "B.Cu") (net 22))
 (segment (start 200.5 95.5) (end 200.5 99.5) (width 0.2032) (layer "B.Cu") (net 22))
 (segment (start 206.25 110) (end 207 110.75) (width 0.2032) (layer "B.Cu") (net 24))
 (segment (start 199.879921 105.632) (end 200.5 106.252079) (width 0.2032) (layer "B.Cu") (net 24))
 (segment (start 199.5 105.632) (end 199.879921 105.632) (width 0.2032) (layer "B.Cu") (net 24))
 (segment (start 201.75 110) (end 206.25 110) (width 0.2032) (layer "B.Cu") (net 24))
 (segment (start 200.5 108.75) (end 201.75 110) (width 0.2032) (layer "B.Cu") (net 24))
 (segment (start 200.5 106.252079) (end 200.5 108.75) (width 0.2032) (layer "B.Cu") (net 24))
 (segment (start 204.718 110.5) (end 200.5 110.5) (width 0.2032) (layer "B.Cu") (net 25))
 (segment (start 207 112.782) (end 204.718 110.5) (width 0.2032) (layer "B.Cu") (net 25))
 (segment (start 200.5 110.5) (end 199.5 109.5) (width 0.2032) (layer "B.Cu") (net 25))
 (segment (start 199.5 109.5) (end 199.5 106.032) (width 0.2032) (layer "B.Cu") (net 25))
 (segment (start 202.75 102.25) (end 202.25 102.25) (width 0.2032) (layer "B.Cu") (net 26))
 (segment (start 200.868 103.632) (end 199.58 103.632) (width 0.2032) (layer "B.Cu") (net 26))
 (segment (start 202.75 100) (end 202.75 102.25) (width 0.2032) (layer "B.Cu") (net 26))
 (segment (start 202.25 102.25) (end 200.868 103.632) (width 0.2032) (layer "B.Cu") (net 26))
 (segment (start 207 108.718) (end 201.968 108.718) (width 0.2032) (layer "B.Cu") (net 28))
 (segment (start 200.75 105.25) (end 199.518 105.25) (width 0.2032) (layer "B.Cu") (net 28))
 (segment (start 199.518 105.25) (end 199.5 105.232) (width 0.2032) (layer "B.Cu") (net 28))
 (segment (start 201 107.75) (end 201 105.5) (width 0.2032) (layer "B.Cu") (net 28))
 (segment (start 201 105.5) (end 200.75 105.25) (width 0.2032) (layer "B.Cu") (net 28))
 (segment (start 201.968 108.718) (end 201 107.75) (width 0.2032) (layer "B.Cu") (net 28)))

